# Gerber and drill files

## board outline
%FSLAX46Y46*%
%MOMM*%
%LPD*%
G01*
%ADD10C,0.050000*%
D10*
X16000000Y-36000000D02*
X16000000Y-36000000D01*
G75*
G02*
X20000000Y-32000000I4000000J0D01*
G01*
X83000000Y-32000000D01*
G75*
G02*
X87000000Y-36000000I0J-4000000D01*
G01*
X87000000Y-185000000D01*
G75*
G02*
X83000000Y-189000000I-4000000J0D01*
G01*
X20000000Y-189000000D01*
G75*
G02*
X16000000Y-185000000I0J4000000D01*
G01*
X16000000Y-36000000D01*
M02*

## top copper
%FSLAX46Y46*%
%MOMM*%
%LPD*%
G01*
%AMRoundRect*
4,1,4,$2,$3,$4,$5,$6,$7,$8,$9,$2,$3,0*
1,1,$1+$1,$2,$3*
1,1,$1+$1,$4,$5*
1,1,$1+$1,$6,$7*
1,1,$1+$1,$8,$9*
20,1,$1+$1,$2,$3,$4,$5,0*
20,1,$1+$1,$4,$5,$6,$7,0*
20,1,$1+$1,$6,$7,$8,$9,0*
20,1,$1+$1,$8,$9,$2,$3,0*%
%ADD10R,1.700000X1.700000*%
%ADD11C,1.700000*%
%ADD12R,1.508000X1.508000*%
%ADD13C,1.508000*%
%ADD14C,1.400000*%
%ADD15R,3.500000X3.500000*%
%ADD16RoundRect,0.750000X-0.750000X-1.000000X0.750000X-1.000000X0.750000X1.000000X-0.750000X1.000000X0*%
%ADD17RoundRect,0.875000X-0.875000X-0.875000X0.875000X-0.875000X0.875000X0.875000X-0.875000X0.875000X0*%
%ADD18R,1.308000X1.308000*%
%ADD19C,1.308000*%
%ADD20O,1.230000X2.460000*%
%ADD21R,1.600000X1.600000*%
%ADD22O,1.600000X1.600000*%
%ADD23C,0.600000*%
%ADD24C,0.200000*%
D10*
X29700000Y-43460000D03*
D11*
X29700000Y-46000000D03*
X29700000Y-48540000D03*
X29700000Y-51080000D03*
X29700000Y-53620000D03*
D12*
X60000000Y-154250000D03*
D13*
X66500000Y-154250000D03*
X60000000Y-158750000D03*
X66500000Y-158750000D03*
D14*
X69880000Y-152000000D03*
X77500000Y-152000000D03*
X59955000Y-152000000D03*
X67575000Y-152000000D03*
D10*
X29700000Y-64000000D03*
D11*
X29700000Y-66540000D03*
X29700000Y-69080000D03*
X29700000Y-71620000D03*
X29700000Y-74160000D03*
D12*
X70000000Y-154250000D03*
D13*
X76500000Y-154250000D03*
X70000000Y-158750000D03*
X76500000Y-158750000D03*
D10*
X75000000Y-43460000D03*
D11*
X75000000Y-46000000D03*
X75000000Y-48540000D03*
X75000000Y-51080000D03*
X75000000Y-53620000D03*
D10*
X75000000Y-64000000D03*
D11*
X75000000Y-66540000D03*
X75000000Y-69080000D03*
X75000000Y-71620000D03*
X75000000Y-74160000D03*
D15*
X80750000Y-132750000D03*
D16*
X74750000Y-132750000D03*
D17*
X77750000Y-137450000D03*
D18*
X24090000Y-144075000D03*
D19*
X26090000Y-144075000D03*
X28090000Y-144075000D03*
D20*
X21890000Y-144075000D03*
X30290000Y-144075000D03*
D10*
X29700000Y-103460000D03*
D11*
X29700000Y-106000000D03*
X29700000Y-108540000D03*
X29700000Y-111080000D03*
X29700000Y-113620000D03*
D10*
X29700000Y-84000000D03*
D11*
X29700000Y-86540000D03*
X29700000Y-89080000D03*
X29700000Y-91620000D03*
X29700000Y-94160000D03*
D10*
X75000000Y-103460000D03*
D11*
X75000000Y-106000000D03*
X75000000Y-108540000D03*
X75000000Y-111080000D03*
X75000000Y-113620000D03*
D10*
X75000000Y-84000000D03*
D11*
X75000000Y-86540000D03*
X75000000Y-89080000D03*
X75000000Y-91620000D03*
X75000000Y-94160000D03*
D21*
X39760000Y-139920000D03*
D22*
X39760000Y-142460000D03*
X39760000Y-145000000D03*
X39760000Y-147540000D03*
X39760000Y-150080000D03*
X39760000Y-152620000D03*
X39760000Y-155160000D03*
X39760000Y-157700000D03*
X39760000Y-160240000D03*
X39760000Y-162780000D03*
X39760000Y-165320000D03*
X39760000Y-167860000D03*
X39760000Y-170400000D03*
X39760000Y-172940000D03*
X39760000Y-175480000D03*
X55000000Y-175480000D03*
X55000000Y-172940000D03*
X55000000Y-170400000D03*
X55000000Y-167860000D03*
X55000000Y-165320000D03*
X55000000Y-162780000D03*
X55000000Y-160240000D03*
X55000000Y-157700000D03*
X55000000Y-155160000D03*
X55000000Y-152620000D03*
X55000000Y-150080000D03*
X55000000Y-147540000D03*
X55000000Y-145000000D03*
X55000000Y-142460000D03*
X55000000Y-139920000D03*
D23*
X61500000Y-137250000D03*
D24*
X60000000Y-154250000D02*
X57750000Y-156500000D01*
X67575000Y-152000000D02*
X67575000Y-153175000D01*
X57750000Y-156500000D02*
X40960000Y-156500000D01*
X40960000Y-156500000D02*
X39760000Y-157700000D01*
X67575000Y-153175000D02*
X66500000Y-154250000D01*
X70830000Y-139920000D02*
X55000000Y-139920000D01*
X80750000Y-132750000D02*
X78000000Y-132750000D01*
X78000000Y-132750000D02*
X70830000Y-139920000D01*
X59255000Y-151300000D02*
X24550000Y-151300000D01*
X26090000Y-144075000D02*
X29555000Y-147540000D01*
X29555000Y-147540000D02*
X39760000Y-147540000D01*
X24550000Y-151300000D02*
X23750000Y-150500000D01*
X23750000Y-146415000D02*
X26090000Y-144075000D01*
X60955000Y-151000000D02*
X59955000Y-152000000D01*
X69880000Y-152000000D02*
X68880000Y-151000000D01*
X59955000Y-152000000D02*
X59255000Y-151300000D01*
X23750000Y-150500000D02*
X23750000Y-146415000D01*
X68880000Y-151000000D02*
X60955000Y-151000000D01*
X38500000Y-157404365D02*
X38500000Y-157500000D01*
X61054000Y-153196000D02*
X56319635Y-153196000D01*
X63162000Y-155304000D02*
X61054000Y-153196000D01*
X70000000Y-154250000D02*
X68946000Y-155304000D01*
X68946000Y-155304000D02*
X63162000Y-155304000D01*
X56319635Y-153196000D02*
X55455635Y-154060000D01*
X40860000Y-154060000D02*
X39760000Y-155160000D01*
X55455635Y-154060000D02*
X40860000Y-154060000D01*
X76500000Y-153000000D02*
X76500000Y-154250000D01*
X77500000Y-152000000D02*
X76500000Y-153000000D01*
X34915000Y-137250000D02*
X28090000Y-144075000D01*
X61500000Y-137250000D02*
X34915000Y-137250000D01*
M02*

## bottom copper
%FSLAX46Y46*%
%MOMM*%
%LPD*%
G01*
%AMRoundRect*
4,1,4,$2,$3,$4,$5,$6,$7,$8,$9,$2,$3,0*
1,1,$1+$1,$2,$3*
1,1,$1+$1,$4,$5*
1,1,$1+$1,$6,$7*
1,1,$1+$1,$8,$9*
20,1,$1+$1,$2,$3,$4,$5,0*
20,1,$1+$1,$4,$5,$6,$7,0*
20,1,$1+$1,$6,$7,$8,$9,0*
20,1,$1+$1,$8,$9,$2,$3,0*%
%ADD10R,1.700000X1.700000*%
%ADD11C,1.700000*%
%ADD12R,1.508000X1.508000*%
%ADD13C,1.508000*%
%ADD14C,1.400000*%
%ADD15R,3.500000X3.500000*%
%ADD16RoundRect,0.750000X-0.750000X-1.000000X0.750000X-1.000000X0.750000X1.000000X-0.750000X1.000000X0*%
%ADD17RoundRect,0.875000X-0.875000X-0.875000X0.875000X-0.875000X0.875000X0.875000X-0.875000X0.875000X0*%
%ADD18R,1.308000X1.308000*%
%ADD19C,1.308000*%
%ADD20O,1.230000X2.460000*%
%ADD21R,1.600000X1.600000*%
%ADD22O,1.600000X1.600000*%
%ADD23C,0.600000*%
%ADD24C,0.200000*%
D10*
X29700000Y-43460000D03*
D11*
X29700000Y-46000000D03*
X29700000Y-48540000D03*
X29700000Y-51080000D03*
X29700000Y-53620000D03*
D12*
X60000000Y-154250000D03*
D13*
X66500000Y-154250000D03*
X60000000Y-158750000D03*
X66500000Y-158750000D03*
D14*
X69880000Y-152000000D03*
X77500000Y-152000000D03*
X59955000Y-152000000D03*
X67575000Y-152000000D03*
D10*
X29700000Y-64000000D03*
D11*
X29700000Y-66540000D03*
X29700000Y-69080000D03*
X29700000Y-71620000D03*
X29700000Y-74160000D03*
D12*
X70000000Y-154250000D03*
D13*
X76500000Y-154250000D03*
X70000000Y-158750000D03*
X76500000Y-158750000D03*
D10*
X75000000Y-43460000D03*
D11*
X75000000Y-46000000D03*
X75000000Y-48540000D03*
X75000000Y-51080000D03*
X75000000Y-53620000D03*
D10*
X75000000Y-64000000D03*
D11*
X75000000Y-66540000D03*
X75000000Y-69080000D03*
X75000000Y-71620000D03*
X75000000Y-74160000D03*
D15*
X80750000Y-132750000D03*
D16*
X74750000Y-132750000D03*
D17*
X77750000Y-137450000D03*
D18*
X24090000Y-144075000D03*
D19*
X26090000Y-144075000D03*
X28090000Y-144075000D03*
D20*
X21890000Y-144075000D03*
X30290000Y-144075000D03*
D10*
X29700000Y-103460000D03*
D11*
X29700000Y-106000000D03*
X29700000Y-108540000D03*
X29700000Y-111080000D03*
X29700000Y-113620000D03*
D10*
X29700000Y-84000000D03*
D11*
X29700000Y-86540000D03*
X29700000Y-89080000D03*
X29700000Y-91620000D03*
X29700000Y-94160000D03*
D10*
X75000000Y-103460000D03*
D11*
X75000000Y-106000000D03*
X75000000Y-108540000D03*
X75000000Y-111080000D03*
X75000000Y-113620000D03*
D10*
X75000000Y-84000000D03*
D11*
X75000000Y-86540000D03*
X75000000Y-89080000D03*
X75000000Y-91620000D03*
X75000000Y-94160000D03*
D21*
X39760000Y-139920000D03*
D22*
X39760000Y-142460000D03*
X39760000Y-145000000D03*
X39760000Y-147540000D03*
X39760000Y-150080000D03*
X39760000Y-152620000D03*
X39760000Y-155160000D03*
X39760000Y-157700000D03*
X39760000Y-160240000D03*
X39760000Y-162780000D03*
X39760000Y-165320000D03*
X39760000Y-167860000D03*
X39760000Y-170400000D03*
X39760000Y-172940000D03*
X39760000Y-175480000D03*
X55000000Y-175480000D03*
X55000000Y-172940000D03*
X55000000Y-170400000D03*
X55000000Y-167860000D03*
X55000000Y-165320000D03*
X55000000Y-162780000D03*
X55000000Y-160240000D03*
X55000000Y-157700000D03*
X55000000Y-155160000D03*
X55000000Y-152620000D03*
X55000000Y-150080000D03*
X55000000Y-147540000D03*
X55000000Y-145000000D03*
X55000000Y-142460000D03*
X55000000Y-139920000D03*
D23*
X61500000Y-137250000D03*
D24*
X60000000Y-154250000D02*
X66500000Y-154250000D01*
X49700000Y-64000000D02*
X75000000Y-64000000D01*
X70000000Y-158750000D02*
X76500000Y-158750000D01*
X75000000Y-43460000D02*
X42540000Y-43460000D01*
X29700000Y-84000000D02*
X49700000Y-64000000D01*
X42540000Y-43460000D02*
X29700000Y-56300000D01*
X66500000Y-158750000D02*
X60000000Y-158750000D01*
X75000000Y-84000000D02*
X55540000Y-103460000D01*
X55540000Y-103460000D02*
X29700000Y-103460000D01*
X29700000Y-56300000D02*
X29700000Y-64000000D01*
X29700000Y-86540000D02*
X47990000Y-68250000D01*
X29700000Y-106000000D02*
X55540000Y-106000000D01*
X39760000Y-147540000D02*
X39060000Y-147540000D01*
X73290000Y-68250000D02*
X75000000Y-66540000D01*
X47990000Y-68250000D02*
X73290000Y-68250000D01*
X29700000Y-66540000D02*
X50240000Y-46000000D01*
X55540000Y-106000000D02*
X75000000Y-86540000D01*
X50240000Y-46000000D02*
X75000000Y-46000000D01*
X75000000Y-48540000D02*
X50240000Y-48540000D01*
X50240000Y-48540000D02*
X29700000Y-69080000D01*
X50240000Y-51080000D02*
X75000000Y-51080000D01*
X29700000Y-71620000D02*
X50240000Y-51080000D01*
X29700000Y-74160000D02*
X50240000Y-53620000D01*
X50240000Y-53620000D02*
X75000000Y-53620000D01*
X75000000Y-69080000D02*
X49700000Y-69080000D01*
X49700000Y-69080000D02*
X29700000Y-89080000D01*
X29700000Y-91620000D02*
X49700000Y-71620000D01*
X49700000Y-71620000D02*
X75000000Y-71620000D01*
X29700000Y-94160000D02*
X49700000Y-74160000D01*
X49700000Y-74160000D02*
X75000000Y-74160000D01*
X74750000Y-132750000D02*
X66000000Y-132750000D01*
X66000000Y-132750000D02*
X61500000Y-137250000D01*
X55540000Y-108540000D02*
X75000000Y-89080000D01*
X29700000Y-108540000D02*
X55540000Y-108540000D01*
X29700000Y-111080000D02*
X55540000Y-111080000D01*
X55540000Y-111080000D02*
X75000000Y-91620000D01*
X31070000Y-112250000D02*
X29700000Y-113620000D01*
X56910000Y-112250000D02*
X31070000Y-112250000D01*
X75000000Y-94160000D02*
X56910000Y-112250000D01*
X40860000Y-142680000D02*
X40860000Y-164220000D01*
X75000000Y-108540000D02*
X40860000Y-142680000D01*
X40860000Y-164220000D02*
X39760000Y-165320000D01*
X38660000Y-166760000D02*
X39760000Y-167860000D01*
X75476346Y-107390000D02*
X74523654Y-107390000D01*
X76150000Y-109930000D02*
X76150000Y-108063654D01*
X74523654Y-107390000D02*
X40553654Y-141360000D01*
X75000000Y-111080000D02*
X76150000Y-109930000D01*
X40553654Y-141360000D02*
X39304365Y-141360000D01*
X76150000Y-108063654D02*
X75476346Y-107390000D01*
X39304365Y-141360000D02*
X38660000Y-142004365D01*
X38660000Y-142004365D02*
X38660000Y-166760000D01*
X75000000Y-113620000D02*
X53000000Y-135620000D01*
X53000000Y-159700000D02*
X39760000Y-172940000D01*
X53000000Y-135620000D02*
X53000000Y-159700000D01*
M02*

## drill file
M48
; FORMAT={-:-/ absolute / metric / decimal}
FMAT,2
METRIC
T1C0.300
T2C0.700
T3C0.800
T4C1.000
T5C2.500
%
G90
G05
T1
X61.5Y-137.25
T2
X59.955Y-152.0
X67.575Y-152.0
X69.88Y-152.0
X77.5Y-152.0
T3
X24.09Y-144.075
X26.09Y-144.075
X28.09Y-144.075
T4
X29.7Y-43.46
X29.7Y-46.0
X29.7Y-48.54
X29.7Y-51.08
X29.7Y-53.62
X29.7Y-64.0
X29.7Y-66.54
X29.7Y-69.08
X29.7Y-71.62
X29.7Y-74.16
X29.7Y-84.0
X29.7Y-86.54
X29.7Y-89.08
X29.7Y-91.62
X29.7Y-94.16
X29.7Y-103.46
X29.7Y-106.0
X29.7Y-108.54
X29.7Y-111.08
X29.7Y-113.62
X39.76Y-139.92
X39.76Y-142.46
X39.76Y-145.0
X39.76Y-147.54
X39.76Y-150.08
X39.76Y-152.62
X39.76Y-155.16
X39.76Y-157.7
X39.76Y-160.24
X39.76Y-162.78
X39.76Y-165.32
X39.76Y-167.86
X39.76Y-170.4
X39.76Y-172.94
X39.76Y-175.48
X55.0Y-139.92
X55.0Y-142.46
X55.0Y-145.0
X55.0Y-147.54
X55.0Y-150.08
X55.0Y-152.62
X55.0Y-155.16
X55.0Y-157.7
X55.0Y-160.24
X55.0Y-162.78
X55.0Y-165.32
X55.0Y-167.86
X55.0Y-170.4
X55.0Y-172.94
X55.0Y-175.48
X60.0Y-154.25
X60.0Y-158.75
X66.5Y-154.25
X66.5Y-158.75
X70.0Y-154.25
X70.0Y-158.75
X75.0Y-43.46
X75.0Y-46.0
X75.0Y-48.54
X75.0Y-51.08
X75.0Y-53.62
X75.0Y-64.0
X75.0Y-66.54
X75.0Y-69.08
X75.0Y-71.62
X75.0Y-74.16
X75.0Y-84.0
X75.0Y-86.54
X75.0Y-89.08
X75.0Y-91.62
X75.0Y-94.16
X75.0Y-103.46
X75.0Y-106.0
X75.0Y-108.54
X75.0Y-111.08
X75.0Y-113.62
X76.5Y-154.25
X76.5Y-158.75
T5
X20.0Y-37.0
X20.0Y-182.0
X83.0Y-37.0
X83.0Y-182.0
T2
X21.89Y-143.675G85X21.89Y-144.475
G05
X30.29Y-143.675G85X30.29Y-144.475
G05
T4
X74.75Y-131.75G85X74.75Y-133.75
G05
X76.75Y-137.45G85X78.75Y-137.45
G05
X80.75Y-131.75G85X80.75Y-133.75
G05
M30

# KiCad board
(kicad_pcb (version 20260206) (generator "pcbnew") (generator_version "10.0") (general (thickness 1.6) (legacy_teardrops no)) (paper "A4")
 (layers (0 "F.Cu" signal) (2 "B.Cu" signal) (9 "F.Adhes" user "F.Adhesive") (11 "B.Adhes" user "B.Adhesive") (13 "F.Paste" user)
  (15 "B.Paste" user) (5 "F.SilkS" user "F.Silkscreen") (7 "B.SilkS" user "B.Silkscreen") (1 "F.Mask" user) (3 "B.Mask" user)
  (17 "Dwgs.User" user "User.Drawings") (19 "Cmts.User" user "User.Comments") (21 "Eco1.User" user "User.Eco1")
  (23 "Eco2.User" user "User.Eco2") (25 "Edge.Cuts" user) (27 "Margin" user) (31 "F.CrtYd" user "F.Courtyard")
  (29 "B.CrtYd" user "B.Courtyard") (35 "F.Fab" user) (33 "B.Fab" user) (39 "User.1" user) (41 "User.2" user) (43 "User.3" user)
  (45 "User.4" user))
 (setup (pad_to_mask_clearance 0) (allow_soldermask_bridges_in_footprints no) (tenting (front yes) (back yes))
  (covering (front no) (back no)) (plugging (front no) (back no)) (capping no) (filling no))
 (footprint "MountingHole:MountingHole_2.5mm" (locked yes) (layer "F.Cu") (at 20 182)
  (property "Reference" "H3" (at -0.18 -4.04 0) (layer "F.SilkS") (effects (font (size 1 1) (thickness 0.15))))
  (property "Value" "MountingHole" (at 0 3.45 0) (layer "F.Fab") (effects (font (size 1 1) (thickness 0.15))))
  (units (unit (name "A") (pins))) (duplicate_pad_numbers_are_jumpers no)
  (pad "" np_thru_hole circle (at 0 0) (size 2.5 2.5) (drill 2.5) (layers "*.Cu" "*.Mask")))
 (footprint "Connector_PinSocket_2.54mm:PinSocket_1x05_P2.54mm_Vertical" (layer "F.Cu") (at 29.7 43.46)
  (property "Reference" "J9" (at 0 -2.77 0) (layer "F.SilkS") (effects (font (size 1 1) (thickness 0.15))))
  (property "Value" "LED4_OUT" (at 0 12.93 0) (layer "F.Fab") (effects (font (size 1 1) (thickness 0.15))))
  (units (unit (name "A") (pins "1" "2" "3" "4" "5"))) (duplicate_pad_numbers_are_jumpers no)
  (pad "1" thru_hole rect (at 0 0) (size 1.7 1.7) (drill 1) (layers "*.Cu" "*.Mask") (remove_unused_layers no)
   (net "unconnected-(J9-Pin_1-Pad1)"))
  (pad "2" thru_hole circle (at 0 2.54) (size 1.7 1.7) (drill 1) (layers "*.Cu" "*.Mask") (remove_unused_layers no)
   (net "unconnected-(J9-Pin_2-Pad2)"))
  (pad "3" thru_hole circle (at 0 5.08) (size 1.7 1.7) (drill 1) (layers "*.Cu" "*.Mask") (remove_unused_layers no)
   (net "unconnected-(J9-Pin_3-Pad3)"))
  (pad "4" thru_hole circle (at 0 7.62) (size 1.7 1.7) (drill 1) (layers "*.Cu" "*.Mask") (remove_unused_layers no)
   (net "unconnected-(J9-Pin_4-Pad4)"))
  (pad "5" thru_hole circle (at 0 10.16) (size 1.7 1.7) (drill 1) (layers "*.Cu" "*.Mask") (remove_unused_layers no)
   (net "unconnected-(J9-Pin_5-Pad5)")))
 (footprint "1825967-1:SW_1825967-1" (layer "F.Cu") (at 63.25 156.5)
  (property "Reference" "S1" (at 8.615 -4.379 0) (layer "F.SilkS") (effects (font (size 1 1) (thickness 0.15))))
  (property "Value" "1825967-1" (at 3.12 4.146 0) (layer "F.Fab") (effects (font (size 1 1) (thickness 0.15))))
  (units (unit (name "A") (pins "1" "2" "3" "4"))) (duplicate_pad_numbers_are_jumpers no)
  (pad "1" thru_hole rect (at -3.25 -2.25) (size 1.508 1.508) (drill 1) (layers "*.Cu" "*.Mask") (remove_unused_layers no)
   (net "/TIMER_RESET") (solder_mask_margin 0.102))
  (pad "2" thru_hole circle (at 3.25 -2.25) (size 1.508 1.508) (drill 1) (layers "*.Cu" "*.Mask") (remove_unused_layers no)
   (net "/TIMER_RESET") (solder_mask_margin 0.102))
  (pad "3" thru_hole circle (at -3.25 2.25) (size 1.508 1.508) (drill 1) (layers "*.Cu" "*.Mask") (remove_unused_layers no) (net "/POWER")
   (solder_mask_margin 0.102))
  (pad "4" thru_hole circle (at 3.25 2.25) (size 1.508 1.508) (drill 1) (layers "*.Cu" "*.Mask") (remove_unused_layers no) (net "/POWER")
   (solder_mask_margin 0.102)))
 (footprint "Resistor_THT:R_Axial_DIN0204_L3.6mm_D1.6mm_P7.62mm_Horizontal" (layer "F.Cu") (at 69.88 152)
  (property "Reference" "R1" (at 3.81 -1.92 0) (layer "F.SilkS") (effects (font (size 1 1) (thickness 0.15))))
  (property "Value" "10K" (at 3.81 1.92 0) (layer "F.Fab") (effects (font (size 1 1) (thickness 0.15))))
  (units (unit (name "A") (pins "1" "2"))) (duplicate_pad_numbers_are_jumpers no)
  (pad "1" thru_hole circle (at 0 0) (size 1.4 1.4) (drill 0.7) (layers "*.Cu" "*.Mask") (remove_unused_layers no) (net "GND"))
  (pad "2" thru_hole circle (at 7.62 0) (size 1.4 1.4) (drill 0.7) (layers "*.Cu" "*.Mask") (remove_unused_layers no) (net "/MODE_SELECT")))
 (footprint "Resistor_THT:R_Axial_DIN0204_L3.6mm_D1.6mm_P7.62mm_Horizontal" (layer "F.Cu") (at 59.955 152)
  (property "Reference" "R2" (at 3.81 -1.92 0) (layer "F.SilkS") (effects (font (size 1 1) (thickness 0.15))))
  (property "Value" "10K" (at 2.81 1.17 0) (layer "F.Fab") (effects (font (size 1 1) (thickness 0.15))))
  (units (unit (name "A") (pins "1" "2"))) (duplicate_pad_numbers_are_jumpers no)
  (pad "1" thru_hole circle (at 0 0) (size 1.4 1.4) (drill 0.7) (layers "*.Cu" "*.Mask") (remove_unused_layers no) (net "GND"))
  (pad "2" thru_hole circle (at 7.62 0) (size 1.4 1.4) (drill 0.7) (layers "*.Cu" "*.Mask") (remove_unused_layers no) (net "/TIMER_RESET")))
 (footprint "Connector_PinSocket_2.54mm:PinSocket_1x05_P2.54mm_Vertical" (layer "F.Cu") (at 29.7 64)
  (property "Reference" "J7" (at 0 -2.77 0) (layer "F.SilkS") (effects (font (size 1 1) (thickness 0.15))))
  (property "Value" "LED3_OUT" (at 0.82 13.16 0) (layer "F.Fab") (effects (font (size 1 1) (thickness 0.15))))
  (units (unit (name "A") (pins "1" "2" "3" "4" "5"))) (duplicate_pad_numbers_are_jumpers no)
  (pad "1" thru_hole rect (at 0 0) (size 1.7 1.7) (drill 1) (layers "*.Cu" "*.Mask") (remove_unused_layers no) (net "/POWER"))
  (pad "2" thru_hole circle (at 0 2.54) (size 1.7 1.7) (drill 1) (layers "*.Cu" "*.Mask") (remove_unused_layers no) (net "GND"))
  (pad "3" thru_hole circle (at 0 5.08) (size 1.7 1.7) (drill 1) (layers "*.Cu" "*.Mask") (remove_unused_layers no) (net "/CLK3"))
  (pad "4" thru_hole circle (at 0 7.62) (size 1.7 1.7) (drill 1) (layers "*.Cu" "*.Mask") (remove_unused_layers no) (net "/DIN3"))
  (pad "5" thru_hole circle (at 0 10.16) (size 1.7 1.7) (drill 1) (layers "*.Cu" "*.Mask") (remove_unused_layers no) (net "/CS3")))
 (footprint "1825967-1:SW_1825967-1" (layer "F.Cu") (at 73.25 156.5)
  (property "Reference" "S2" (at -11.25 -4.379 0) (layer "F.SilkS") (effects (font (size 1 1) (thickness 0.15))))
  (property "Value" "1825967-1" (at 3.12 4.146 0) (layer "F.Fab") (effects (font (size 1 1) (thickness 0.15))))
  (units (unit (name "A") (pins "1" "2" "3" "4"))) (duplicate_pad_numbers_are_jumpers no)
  (pad "1" thru_hole rect (at -3.25 -2.25) (size 1.508 1.508) (drill 1) (layers "*.Cu" "*.Mask") (remove_unused_layers no)
   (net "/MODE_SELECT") (solder_mask_margin 0.102))
  (pad "2" thru_hole circle (at 3.25 -2.25) (size 1.508 1.508) (drill 1) (layers "*.Cu" "*.Mask") (remove_unused_layers no)
   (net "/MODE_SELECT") (solder_mask_margin 0.102))
  (pad "3" thru_hole circle (at -3.25 2.25) (size 1.508 1.508) (drill 1) (layers "*.Cu" "*.Mask") (remove_unused_layers no) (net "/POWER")
   (solder_mask_margin 0.102))
  (pad "4" thru_hole circle (at 3.25 2.25) (size 1.508 1.508) (drill 1) (layers "*.Cu" "*.Mask") (remove_unused_layers no) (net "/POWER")
   (solder_mask_margin 0.102)))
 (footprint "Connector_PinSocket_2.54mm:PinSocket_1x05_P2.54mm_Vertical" (layer "F.Cu") (at 75 43.46)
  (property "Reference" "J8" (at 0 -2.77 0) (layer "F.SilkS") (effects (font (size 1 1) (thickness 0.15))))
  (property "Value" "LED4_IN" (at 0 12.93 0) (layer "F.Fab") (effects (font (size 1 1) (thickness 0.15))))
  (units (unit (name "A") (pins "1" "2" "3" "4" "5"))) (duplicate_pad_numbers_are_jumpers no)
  (pad "1" thru_hole rect (at 0 0) (size 1.7 1.7) (drill 1) (layers "*.Cu" "*.Mask") (remove_unused_layers no) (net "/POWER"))
  (pad "2" thru_hole circle (at 0 2.54) (size 1.7 1.7) (drill 1) (layers "*.Cu" "*.Mask") (remove_unused_layers no) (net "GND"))
  (pad "3" thru_hole circle (at 0 5.08) (size 1.7 1.7) (drill 1) (layers "*.Cu" "*.Mask") (remove_unused_layers no) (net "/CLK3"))
  (pad "4" thru_hole circle (at 0 7.62) (size 1.7 1.7) (drill 1) (layers "*.Cu" "*.Mask") (remove_unused_layers no) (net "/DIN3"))
  (pad "5" thru_hole circle (at 0 10.16) (size 1.7 1.7) (drill 1) (layers "*.Cu" "*.Mask") (remove_unused_layers no) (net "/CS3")))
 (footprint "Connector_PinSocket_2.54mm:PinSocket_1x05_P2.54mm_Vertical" (layer "F.Cu") (at 75 64)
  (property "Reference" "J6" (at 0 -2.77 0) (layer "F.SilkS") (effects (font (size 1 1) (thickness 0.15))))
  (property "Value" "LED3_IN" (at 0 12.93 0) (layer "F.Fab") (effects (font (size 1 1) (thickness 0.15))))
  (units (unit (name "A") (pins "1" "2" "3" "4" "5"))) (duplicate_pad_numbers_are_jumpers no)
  (pad "1" thru_hole rect (at 0 0) (size 1.7 1.7) (drill 1) (layers "*.Cu" "*.Mask") (remove_unused_layers no) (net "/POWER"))
  (pad "2" thru_hole circle (at 0 2.54) (size 1.7 1.7) (drill 1) (layers "*.Cu" "*.Mask") (remove_unused_layers no) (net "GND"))
  (pad "3" thru_hole circle (at 0 5.08) (size 1.7 1.7) (drill 1) (layers "*.Cu" "*.Mask") (remove_unused_layers no) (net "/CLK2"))
  (pad "4" thru_hole circle (at 0 7.62) (size 1.7 1.7) (drill 1) (layers "*.Cu" "*.Mask") (remove_unused_layers no) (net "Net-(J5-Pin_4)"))
  (pad "5" thru_hole circle (at 0 10.16) (size 1.7 1.7) (drill 1) (layers "*.Cu" "*.Mask") (remove_unused_layers no) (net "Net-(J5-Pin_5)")))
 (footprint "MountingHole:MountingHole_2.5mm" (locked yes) (layer "F.Cu") (at 83 182)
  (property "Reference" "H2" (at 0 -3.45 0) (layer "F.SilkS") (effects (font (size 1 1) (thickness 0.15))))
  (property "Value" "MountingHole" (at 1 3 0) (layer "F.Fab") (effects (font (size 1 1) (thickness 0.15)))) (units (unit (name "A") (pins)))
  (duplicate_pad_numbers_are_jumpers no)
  (pad "" np_thru_hole circle (at 0 0) (size 2.5 2.5) (drill 2.5) (layers "*.Cu" "*.Mask")))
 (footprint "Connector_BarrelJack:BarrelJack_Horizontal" (layer "F.Cu") (at 80.75 132.75)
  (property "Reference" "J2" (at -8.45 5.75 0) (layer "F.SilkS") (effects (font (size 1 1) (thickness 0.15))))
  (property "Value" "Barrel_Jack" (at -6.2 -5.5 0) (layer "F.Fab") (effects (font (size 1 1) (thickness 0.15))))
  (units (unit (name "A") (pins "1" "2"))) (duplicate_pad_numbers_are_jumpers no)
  (pad "1" thru_hole rect (at 0 0) (size 3.5 3.5) (drill oval 1 3) (layers "*.Cu" "*.Mask") (remove_unused_layers no) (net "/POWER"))
  (pad "2" thru_hole roundrect (at -6 0) (size 3 3.5) (drill oval 1 3) (layers "*.Cu" "*.Mask") (remove_unused_layers no)
   (roundrect_rratio 0.25) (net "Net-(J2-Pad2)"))
  (pad "3" thru_hole roundrect (at -3 4.7) (size 3.5 3.5) (drill oval 3 1) (layers "*.Cu" "*.Mask") (remove_unused_layers no)
   (roundrect_rratio 0.25)))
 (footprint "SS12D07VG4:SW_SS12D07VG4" (layer "F.Cu") (at 26.09 144.075)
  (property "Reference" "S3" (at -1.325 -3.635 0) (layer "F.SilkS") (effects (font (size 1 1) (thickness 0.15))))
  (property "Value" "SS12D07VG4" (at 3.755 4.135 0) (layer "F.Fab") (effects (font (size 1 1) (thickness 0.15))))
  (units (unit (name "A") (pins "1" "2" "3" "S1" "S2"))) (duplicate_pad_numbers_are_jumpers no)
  (pad "1" thru_hole rect (at -2 0) (size 1.308 1.308) (drill 0.8) (layers "*.Cu" "*.Mask") (remove_unused_layers no)
   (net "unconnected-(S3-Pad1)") (solder_mask_margin 0.102))
  (pad "2" thru_hole circle (at 0 0) (size 1.308 1.308) (drill 0.8) (layers "*.Cu" "*.Mask") (remove_unused_layers no) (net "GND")
   (solder_mask_margin 0.102))
  (pad "3" thru_hole circle (at 2 0) (size 1.308 1.308) (drill 0.8) (layers "*.Cu" "*.Mask") (remove_unused_layers no) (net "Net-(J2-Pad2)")
   (solder_mask_margin 0.102))
  (pad "S1" thru_hole oval (at -4.2 0) (size 1.23 2.46) (drill oval 0.7 1.5) (layers "*.Cu" "*.Mask") (remove_unused_layers no)
   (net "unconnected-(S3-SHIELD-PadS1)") (solder_mask_margin 0.102))
  (pad "S2" thru_hole oval (at 4.2 0) (size 1.23 2.46) (drill oval 0.7 1.5) (layers "*.Cu" "*.Mask") (remove_unused_layers no)
   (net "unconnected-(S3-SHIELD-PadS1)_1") (solder_mask_margin 0.102)))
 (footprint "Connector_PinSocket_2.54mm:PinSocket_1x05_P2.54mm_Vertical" (layer "F.Cu") (at 29.7 103.46)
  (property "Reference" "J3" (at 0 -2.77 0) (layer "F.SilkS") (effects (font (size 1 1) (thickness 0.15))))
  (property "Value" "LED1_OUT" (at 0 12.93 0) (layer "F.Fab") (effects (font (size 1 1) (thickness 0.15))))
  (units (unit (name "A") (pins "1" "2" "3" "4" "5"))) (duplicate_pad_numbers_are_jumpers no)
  (pad "1" thru_hole rect (at 0 0) (size 1.7 1.7) (drill 1) (layers "*.Cu" "*.Mask") (remove_unused_layers no) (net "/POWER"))
  (pad "2" thru_hole circle (at 0 2.54) (size 1.7 1.7) (drill 1) (layers "*.Cu" "*.Mask") (remove_unused_layers no) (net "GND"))
  (pad "3" thru_hole circle (at 0 5.08) (size 1.7 1.7) (drill 1) (layers "*.Cu" "*.Mask") (remove_unused_layers no) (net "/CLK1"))
  (pad "4" thru_hole circle (at 0 7.62) (size 1.7 1.7) (drill 1) (layers "*.Cu" "*.Mask") (remove_unused_layers no) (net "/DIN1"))
  (pad "5" thru_hole circle (at 0 10.16) (size 1.7 1.7) (drill 1) (layers "*.Cu" "*.Mask") (remove_unused_layers no) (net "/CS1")))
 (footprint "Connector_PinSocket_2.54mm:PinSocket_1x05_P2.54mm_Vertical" (layer "F.Cu") (at 29.7 84)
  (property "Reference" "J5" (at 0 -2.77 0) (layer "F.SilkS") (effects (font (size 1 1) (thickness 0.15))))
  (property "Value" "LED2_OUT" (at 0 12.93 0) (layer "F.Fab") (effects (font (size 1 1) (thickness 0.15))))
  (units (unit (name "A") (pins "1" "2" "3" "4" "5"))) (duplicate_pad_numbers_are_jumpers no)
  (pad "1" thru_hole rect (at 0 0) (size 1.7 1.7) (drill 1) (layers "*.Cu" "*.Mask") (remove_unused_layers no) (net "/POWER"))
  (pad "2" thru_hole circle (at 0 2.54) (size 1.7 1.7) (drill 1) (layers "*.Cu" "*.Mask") (remove_unused_layers no) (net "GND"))
  (pad "3" thru_hole circle (at 0 5.08) (size 1.7 1.7) (drill 1) (layers "*.Cu" "*.Mask") (remove_unused_layers no) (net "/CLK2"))
  (pad "4" thru_hole circle (at 0 7.62) (size 1.7 1.7) (drill 1) (layers "*.Cu" "*.Mask") (remove_unused_layers no) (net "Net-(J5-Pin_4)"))
  (pad "5" thru_hole circle (at 0 10.16) (size 1.7 1.7) (drill 1) (layers "*.Cu" "*.Mask") (remove_unused_layers no) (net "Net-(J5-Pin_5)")))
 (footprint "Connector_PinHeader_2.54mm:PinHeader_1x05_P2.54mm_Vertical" (layer "F.Cu") (at 75 103.46)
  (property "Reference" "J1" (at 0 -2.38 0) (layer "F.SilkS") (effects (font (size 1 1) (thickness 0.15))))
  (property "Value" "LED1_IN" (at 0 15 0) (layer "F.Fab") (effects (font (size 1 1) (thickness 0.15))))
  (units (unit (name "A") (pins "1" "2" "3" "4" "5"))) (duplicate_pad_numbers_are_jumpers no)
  (pad "1" thru_hole rect (at 0 0) (size 1.7 1.7) (drill 1) (layers "*.Cu" "*.Mask") (remove_unused_layers no)
   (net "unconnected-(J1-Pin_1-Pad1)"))
  (pad "2" thru_hole circle (at 0 2.54) (size 1.7 1.7) (drill 1) (layers "*.Cu" "*.Mask") (remove_unused_layers no)
   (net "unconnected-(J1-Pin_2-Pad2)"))
  (pad "3" thru_hole circle (at 0 5.08) (size 1.7 1.7) (drill 1) (layers "*.Cu" "*.Mask") (remove_unused_layers no) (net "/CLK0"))
  (pad "4" thru_hole circle (at 0 7.62) (size 1.7 1.7) (drill 1) (layers "*.Cu" "*.Mask") (remove_unused_layers no) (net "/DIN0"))
  (pad "5" thru_hole circle (at 0 10.16) (size 1.7 1.7) (drill 1) (layers "*.Cu" "*.Mask") (remove_unused_layers no) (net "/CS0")))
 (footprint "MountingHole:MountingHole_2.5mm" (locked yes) (layer "F.Cu") (at 20 37)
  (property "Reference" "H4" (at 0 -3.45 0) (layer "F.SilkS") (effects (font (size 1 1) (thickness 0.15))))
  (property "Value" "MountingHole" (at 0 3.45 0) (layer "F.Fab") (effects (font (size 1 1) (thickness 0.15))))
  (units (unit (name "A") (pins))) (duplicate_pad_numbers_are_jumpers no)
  (pad "" np_thru_hole circle (at 0 0) (size 2.5 2.5) (drill 2.5) (layers "*.Cu" "*.Mask")))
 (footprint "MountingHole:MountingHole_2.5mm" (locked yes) (layer "F.Cu") (at 83 37)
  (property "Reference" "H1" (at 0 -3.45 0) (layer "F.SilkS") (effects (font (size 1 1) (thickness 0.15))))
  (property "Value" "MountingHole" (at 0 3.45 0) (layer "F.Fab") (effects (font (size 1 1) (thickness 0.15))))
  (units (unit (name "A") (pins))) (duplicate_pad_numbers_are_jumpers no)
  (pad "" np_thru_hole circle (at 0 0) (size 2.5 2.5) (drill 2.5) (layers "*.Cu" "*.Mask")))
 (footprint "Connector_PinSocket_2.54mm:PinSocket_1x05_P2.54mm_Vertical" (layer "F.Cu") (at 75 84)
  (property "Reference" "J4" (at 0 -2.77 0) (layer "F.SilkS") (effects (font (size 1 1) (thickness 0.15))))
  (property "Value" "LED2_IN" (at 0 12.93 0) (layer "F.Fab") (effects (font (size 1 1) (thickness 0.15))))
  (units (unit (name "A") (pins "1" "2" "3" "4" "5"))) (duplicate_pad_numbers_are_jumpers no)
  (pad "1" thru_hole rect (at 0 0) (size 1.7 1.7) (drill 1) (layers "*.Cu" "*.Mask") (remove_unused_layers no) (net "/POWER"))
  (pad "2" thru_hole circle (at 0 2.54) (size 1.7 1.7) (drill 1) (layers "*.Cu" "*.Mask") (remove_unused_layers no) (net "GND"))
  (pad "3" thru_hole circle (at 0 5.08) (size 1.7 1.7) (drill 1) (layers "*.Cu" "*.Mask") (remove_unused_layers no) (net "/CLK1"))
  (pad "4" thru_hole circle (at 0 7.62) (size 1.7 1.7) (drill 1) (layers "*.Cu" "*.Mask") (remove_unused_layers no) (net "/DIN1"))
  (pad "5" thru_hole circle (at 0 10.16) (size 1.7 1.7) (drill 1) (layers "*.Cu" "*.Mask") (remove_unused_layers no) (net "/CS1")))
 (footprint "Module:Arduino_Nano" (layer "F.Cu") (at 39.76 139.92)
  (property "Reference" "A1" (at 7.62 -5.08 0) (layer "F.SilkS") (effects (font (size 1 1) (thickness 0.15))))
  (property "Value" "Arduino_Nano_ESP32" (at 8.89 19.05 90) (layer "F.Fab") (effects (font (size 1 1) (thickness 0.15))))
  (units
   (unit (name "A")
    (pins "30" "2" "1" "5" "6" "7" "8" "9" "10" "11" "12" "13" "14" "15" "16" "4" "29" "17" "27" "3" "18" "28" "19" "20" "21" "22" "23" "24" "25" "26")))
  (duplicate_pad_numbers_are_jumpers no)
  (pad "1" thru_hole rect (at 0 0) (size 1.6 1.6) (drill 1) (layers "*.Cu" "*.Mask") (remove_unused_layers no)
   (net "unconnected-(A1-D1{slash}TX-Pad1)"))
  (pad "2" thru_hole oval (at 0 2.54) (size 1.6 1.6) (drill 1) (layers "*.Cu" "*.Mask") (remove_unused_layers no)
   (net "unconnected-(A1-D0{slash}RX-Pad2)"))
  (pad "3" thru_hole oval (at 0 5.08) (size 1.6 1.6) (drill 1) (layers "*.Cu" "*.Mask") (remove_unused_layers no)
   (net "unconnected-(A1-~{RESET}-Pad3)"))
  (pad "4" thru_hole oval (at 0 7.62) (size 1.6 1.6) (drill 1) (layers "*.Cu" "*.Mask") (remove_unused_layers no) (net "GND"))
  (pad "5" thru_hole oval (at 0 10.16) (size 1.6 1.6) (drill 1) (layers "*.Cu" "*.Mask") (remove_unused_layers no)
   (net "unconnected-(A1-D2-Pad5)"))
  (pad "6" thru_hole oval (at 0 12.7) (size 1.6 1.6) (drill 1) (layers "*.Cu" "*.Mask") (remove_unused_layers no)
   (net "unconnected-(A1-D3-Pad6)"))
  (pad "7" thru_hole oval (at 0 15.24) (size 1.6 1.6) (drill 1) (layers "*.Cu" "*.Mask") (remove_unused_layers no) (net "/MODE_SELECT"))
  (pad "8" thru_hole oval (at 0 17.78) (size 1.6 1.6) (drill 1) (layers "*.Cu" "*.Mask") (remove_unused_layers no) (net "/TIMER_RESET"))
  (pad "9" thru_hole oval (at 0 20.32) (size 1.6 1.6) (drill 1) (layers "*.Cu" "*.Mask") (remove_unused_layers no)
   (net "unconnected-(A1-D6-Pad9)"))
  (pad "10" thru_hole oval (at 0 22.86) (size 1.6 1.6) (drill 1) (layers "*.Cu" "*.Mask") (remove_unused_layers no)
   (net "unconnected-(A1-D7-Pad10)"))
  (pad "11" thru_hole oval (at 0 25.4) (size 1.6 1.6) (drill 1) (layers "*.Cu" "*.Mask") (remove_unused_layers no) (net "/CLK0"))
  (pad "12" thru_hole oval (at 0 27.94) (size 1.6 1.6) (drill 1) (layers "*.Cu" "*.Mask") (remove_unused_layers no) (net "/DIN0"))
  (pad "13" thru_hole oval (at 0 30.48) (size 1.6 1.6) (drill 1) (layers "*.Cu" "*.Mask") (remove_unused_layers no)
   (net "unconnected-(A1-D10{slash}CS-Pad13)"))
  (pad "14" thru_hole oval (at 0 33.02) (size 1.6 1.6) (drill 1) (layers "*.Cu" "*.Mask") (remove_unused_layers no) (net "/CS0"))
  (pad "15" thru_hole oval (at 0 35.56) (size 1.6 1.6) (drill 1) (layers "*.Cu" "*.Mask") (remove_unused_layers no)
   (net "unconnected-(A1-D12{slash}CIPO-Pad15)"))
  (pad "16" thru_hole oval (at 15.24 35.56) (size 1.6 1.6) (drill 1) (layers "*.Cu" "*.Mask") (remove_unused_layers no)
   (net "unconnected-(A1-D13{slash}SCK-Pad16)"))
  (pad "17" thru_hole oval (at 15.24 33.02) (size 1.6 1.6) (drill 1) (layers "*.Cu" "*.Mask") (remove_unused_layers no)
   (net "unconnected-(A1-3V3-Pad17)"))
  (pad "18" thru_hole oval (at 15.24 30.48) (size 1.6 1.6) (drill 1) (layers "*.Cu" "*.Mask") (remove_unused_layers no)
   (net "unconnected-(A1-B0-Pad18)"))
  (pad "19" thru_hole oval (at 15.24 27.94) (size 1.6 1.6) (drill 1) (layers "*.Cu" "*.Mask") (remove_unused_layers no)
   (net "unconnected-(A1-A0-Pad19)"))
  (pad "20" thru_hole oval (at 15.24 25.4) (size 1.6 1.6) (drill 1) (layers "*.Cu" "*.Mask") (remove_unused_layers no)
   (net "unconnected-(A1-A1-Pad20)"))
  (pad "21" thru_hole oval (at 15.24 22.86) (size 1.6 1.6) (drill 1) (layers "*.Cu" "*.Mask") (remove_unused_layers no)
   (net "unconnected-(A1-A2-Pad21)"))
  (pad "22" thru_hole oval (at 15.24 20.32) (size 1.6 1.6) (drill 1) (layers "*.Cu" "*.Mask") (remove_unused_layers no)
   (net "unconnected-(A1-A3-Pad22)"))
  (pad "23" thru_hole oval (at 15.24 17.78) (size 1.6 1.6) (drill 1) (layers "*.Cu" "*.Mask") (remove_unused_layers no)
   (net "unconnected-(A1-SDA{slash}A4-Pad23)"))
  (pad "24" thru_hole oval (at 15.24 15.24) (size 1.6 1.6) (drill 1) (layers "*.Cu" "*.Mask") (remove_unused_layers no)
   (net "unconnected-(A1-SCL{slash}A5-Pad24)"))
  (pad "25" thru_hole oval (at 15.24 12.7) (size 1.6 1.6) (drill 1) (layers "*.Cu" "*.Mask") (remove_unused_layers no)
   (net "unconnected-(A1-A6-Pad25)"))
  (pad "26" thru_hole oval (at 15.24 10.16) (size 1.6 1.6) (drill 1) (layers "*.Cu" "*.Mask") (remove_unused_layers no)
   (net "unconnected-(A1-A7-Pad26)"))
  (pad "27" thru_hole oval (at 15.24 7.62) (size 1.6 1.6) (drill 1) (layers "*.Cu" "*.Mask") (remove_unused_layers no)
   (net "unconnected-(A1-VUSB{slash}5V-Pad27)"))
  (pad "28" thru_hole oval (at 15.24 5.08) (size 1.6 1.6) (drill 1) (layers "*.Cu" "*.Mask") (remove_unused_layers no)
   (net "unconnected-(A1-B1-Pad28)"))
  (pad "29" thru_hole oval (at 15.24 2.54) (size 1.6 1.6) (drill 1) (layers "*.Cu" "*.Mask") (remove_unused_layers no) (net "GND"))
  (pad "30" thru_hole oval (at 15.24 0) (size 1.6 1.6) (drill 1) (layers "*.Cu" "*.Mask") (remove_unused_layers no) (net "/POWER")))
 (gr_rect (start 16 32) (end 87 189) (radius 4) (stroke (width 0.05) (type default)) (fill no) (layer "Edge.Cuts"))
 (segment (start 60 154.25) (end 57.75 156.5) (width 0.2) (layer "F.Cu") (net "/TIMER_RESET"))
 (segment (start 67.575 152) (end 67.575 153.175) (width 0.2) (layer "F.Cu") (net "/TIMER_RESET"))
 (segment (start 57.75 156.5) (end 40.96 156.5) (width 0.2) (layer "F.Cu") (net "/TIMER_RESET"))
 (segment (start 40.96 156.5) (end 39.76 157.7) (width 0.2) (layer "F.Cu") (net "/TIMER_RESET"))
 (segment (start 67.575 153.175) (end 66.5 154.25) (width 0.2) (layer "F.Cu") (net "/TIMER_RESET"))
 (segment (start 60 154.25) (end 66.5 154.25) (width 0.2) (layer "B.Cu") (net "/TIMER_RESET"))
 (segment (start 70.83 139.92) (end 55 139.92) (width 0.2) (layer "F.Cu") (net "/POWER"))
 (segment (start 80.75 132.75) (end 78 132.75) (width 0.2) (layer "F.Cu") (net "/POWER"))
 (segment (start 78 132.75) (end 70.83 139.92) (width 0.2) (layer "F.Cu") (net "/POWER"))
 (segment (start 49.7 64) (end 75 64) (width 0.2) (layer "B.Cu") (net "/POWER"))
 (segment (start 70 158.75) (end 76.5 158.75) (width 0.2) (layer "B.Cu") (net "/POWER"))
 (segment (start 75 43.46) (end 42.54 43.46) (width 0.2) (layer "B.Cu") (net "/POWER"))
 (segment (start 29.7 84) (end 49.7 64) (width 0.2) (layer "B.Cu") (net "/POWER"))
 (segment (start 42.54 43.46) (end 29.7 56.3) (width 0.2) (layer "B.Cu") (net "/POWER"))
 (segment (start 66.5 158.75) (end 60 158.75) (width 0.2) (layer "B.Cu") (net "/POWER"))
 (segment (start 75 84) (end 55.54 103.46) (width 0.2) (layer "B.Cu") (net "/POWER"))
 (segment (start 55.54 103.46) (end 29.7 103.46) (width 0.2) (layer "B.Cu") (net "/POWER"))
 (segment (start 29.7 56.3) (end 29.7 64) (width 0.2) (layer "B.Cu") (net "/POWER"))
 (segment (start 59.255 151.3) (end 24.55 151.3) (width 0.2) (layer "F.Cu") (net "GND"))
 (segment (start 26.09 144.075) (end 29.555 147.54) (width 0.2) (layer "F.Cu") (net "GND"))
 (segment (start 29.555 147.54) (end 39.76 147.54) (width 0.2) (layer "F.Cu") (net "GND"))
 (segment (start 24.55 151.3) (end 23.75 150.5) (width 0.2) (layer "F.Cu") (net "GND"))
 (segment (start 23.75 146.415) (end 26.09 144.075) (width 0.2) (layer "F.Cu") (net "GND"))
 (segment (start 60.955 151) (end 59.955 152) (width 0.2) (layer "F.Cu") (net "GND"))
 (segment (start 69.88 152) (end 68.88 151) (width 0.2) (layer "F.Cu") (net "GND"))
 (segment (start 59.955 152) (end 59.255 151.3) (width 0.2) (layer "F.Cu") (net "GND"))
 (segment (start 23.75 150.5) (end 23.75 146.415) (width 0.2) (layer "F.Cu") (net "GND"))
 (segment (start 68.88 151) (end 60.955 151) (width 0.2) (layer "F.Cu") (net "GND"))
 (segment (start 29.7 86.54) (end 47.99 68.25) (width 0.2) (layer "B.Cu") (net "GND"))
 (segment (start 29.7 106) (end 55.54 106) (width 0.2) (layer "B.Cu") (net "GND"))
 (segment (start 39.76 147.54) (end 39.06 147.54) (width 0.2) (layer "B.Cu") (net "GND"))
 (segment (start 73.29 68.25) (end 75 66.54) (width 0.2) (layer "B.Cu") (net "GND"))
 (segment (start 47.99 68.25) (end 73.29 68.25) (width 0.2) (layer "B.Cu") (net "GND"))
 (segment (start 29.7 66.54) (end 50.24 46) (width 0.2) (layer "B.Cu") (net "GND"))
 (segment (start 55.54 106) (end 75 86.54) (width 0.2) (layer "B.Cu") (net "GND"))
 (segment (start 50.24 46) (end 75 46) (width 0.2) (layer "B.Cu") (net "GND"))
 (segment (start 38.5 157.404365) (end 38.5 157.5) (width 0.2) (layer "F.Cu") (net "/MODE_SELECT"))
 (segment (start 61.054 153.196) (end 56.319635 153.196) (width 0.2) (layer "F.Cu") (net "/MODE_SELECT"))
 (segment (start 63.162 155.304) (end 61.054 153.196) (width 0.2) (layer "F.Cu") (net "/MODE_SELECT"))
 (segment (start 70 154.25) (end 68.946 155.304) (width 0.2) (layer "F.Cu") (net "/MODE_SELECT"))
 (segment (start 68.946 155.304) (end 63.162 155.304) (width 0.2) (layer "F.Cu") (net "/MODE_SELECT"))
 (segment (start 56.319635 153.196) (end 55.455635 154.06) (width 0.2) (layer "F.Cu") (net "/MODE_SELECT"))
 (segment (start 40.86 154.06) (end 39.76 155.16) (width 0.2) (layer "F.Cu") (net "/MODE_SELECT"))
 (segment (start 55.455635 154.06) (end 40.86 154.06) (width 0.2) (layer "F.Cu") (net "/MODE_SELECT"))
 (segment (start 76.5 153) (end 76.5 154.25) (width 0.2) (layer "F.Cu") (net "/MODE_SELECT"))
 (segment (start 77.5 152) (end 76.5 153) (width 0.2) (layer "F.Cu") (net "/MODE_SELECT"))
 (segment (start 75 48.54) (end 50.24 48.54) (width 0.2) (layer "B.Cu") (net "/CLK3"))
 (segment (start 50.24 48.54) (end 29.7 69.08) (width 0.2) (layer "B.Cu") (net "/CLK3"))
 (segment (start 50.24 51.08) (end 75 51.08) (width 0.2) (layer "B.Cu") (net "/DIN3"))
 (segment (start 29.7 71.62) (end 50.24 51.08) (width 0.2) (layer "B.Cu") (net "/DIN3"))
 (segment (start 29.7 74.16) (end 50.24 53.62) (width 0.2) (layer "B.Cu") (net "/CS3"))
 (segment (start 50.24 53.62) (end 75 53.62) (width 0.2) (layer "B.Cu") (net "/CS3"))
 (segment (start 75 69.08) (end 49.7 69.08) (width 0.2) (layer "B.Cu") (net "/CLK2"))
 (segment (start 49.7 69.08) (end 29.7 89.08) (width 0.2) (layer "B.Cu") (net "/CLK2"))
 (segment (start 29.7 91.62) (end 49.7 71.62) (width 0.2) (layer "B.Cu") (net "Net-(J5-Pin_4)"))
 (segment (start 49.7 71.62) (end 75 71.62) (width 0.2) (layer "B.Cu") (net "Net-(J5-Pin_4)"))
 (segment (start 29.7 94.16) (end 49.7 74.16) (width 0.2) (layer "B.Cu") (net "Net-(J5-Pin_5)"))
 (segment (start 49.7 74.16) (end 75 74.16) (width 0.2) (layer "B.Cu") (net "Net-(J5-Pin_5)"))
 (segment (start 34.915 137.25) (end 28.09 144.075) (width 0.2) (layer "F.Cu") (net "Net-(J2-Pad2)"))
 (segment (start 61.5 137.25) (end 34.915 137.25) (width 0.2) (layer "F.Cu") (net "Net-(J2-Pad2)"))
 (via (at 61.5 137.25) (size 0.6) (drill 0.3) (layers "F.Cu" "B.Cu") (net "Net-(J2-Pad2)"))
 (segment (start 74.75 132.75) (end 66 132.75) (width 0.2) (layer "B.Cu") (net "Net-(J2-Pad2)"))
 (segment (start 66 132.75) (end 61.5 137.25) (width 0.2) (layer "B.Cu") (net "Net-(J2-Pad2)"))
 (segment (start 55.54 108.54) (end 75 89.08) (width 0.2) (layer "B.Cu") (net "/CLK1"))
 (segment (start 29.7 108.54) (end 55.54 108.54) (width 0.2) (layer "B.Cu") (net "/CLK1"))
 (segment (start 29.7 111.08) (end 55.54 111.08) (width 0.2) (layer "B.Cu") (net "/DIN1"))
 (segment (start 55.54 111.08) (end 75 91.62) (width 0.2) (layer "B.Cu") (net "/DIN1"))
 (segment (start 31.07 112.25) (end 29.7 113.62) (width 0.2) (layer "B.Cu") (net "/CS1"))
 (segment (start 56.91 112.25) (end 31.07 112.25) (width 0.2) (layer "B.Cu") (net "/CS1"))
 (segment (start 75 94.16) (end 56.91 112.25) (width 0.2) (layer "B.Cu") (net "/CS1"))
 (segment (start 40.86 142.68) (end 40.86 164.22) (width 0.2) (layer "B.Cu") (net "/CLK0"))
 (segment (start 75 108.54) (end 40.86 142.68) (width 0.2) (layer "B.Cu") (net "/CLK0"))
 (segment (start 40.86 164.22) (end 39.76 165.32) (width 0.2) (layer "B.Cu") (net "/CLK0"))
 (segment (start 38.66 166.76) (end 39.76 167.86) (width 0.2) (layer "B.Cu") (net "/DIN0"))
 (segment (start 75.476346 107.39) (end 74.523654 107.39) (width 0.2) (layer "B.Cu") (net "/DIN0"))
 (segment (start 76.15 109.93) (end 76.15 108.063654) (width 0.2) (layer "B.Cu") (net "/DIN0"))
 (segment (start 74.523654 107.39) (end 40.553654 141.36) (width 0.2) (layer "B.Cu") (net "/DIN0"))
 (segment (start 75 111.08) (end 76.15 109.93) (width 0.2) (layer "B.Cu") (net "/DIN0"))
 (segment (start 40.553654 141.36) (end 39.304365 141.36) (width 0.2) (layer "B.Cu") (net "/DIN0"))
 (segment (start 76.15 108.063654) (end 75.476346 107.39) (width 0.2) (layer "B.Cu") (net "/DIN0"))
 (segment (start 39.304365 141.36) (end 38.66 142.004365) (width 0.2) (layer "B.Cu") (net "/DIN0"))
 (segment (start 38.66 142.004365) (end 38.66 166.76) (width 0.2) (layer "B.Cu") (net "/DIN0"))
 (segment (start 75 113.62) (end 53 135.62) (width 0.2) (layer "B.Cu") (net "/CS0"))
 (segment (start 53 159.7) (end 39.76 172.94) (width 0.2) (layer "B.Cu") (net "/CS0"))
 (segment (start 53 135.62) (end 53 159.7) (width 0.2) (layer "B.Cu") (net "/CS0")))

